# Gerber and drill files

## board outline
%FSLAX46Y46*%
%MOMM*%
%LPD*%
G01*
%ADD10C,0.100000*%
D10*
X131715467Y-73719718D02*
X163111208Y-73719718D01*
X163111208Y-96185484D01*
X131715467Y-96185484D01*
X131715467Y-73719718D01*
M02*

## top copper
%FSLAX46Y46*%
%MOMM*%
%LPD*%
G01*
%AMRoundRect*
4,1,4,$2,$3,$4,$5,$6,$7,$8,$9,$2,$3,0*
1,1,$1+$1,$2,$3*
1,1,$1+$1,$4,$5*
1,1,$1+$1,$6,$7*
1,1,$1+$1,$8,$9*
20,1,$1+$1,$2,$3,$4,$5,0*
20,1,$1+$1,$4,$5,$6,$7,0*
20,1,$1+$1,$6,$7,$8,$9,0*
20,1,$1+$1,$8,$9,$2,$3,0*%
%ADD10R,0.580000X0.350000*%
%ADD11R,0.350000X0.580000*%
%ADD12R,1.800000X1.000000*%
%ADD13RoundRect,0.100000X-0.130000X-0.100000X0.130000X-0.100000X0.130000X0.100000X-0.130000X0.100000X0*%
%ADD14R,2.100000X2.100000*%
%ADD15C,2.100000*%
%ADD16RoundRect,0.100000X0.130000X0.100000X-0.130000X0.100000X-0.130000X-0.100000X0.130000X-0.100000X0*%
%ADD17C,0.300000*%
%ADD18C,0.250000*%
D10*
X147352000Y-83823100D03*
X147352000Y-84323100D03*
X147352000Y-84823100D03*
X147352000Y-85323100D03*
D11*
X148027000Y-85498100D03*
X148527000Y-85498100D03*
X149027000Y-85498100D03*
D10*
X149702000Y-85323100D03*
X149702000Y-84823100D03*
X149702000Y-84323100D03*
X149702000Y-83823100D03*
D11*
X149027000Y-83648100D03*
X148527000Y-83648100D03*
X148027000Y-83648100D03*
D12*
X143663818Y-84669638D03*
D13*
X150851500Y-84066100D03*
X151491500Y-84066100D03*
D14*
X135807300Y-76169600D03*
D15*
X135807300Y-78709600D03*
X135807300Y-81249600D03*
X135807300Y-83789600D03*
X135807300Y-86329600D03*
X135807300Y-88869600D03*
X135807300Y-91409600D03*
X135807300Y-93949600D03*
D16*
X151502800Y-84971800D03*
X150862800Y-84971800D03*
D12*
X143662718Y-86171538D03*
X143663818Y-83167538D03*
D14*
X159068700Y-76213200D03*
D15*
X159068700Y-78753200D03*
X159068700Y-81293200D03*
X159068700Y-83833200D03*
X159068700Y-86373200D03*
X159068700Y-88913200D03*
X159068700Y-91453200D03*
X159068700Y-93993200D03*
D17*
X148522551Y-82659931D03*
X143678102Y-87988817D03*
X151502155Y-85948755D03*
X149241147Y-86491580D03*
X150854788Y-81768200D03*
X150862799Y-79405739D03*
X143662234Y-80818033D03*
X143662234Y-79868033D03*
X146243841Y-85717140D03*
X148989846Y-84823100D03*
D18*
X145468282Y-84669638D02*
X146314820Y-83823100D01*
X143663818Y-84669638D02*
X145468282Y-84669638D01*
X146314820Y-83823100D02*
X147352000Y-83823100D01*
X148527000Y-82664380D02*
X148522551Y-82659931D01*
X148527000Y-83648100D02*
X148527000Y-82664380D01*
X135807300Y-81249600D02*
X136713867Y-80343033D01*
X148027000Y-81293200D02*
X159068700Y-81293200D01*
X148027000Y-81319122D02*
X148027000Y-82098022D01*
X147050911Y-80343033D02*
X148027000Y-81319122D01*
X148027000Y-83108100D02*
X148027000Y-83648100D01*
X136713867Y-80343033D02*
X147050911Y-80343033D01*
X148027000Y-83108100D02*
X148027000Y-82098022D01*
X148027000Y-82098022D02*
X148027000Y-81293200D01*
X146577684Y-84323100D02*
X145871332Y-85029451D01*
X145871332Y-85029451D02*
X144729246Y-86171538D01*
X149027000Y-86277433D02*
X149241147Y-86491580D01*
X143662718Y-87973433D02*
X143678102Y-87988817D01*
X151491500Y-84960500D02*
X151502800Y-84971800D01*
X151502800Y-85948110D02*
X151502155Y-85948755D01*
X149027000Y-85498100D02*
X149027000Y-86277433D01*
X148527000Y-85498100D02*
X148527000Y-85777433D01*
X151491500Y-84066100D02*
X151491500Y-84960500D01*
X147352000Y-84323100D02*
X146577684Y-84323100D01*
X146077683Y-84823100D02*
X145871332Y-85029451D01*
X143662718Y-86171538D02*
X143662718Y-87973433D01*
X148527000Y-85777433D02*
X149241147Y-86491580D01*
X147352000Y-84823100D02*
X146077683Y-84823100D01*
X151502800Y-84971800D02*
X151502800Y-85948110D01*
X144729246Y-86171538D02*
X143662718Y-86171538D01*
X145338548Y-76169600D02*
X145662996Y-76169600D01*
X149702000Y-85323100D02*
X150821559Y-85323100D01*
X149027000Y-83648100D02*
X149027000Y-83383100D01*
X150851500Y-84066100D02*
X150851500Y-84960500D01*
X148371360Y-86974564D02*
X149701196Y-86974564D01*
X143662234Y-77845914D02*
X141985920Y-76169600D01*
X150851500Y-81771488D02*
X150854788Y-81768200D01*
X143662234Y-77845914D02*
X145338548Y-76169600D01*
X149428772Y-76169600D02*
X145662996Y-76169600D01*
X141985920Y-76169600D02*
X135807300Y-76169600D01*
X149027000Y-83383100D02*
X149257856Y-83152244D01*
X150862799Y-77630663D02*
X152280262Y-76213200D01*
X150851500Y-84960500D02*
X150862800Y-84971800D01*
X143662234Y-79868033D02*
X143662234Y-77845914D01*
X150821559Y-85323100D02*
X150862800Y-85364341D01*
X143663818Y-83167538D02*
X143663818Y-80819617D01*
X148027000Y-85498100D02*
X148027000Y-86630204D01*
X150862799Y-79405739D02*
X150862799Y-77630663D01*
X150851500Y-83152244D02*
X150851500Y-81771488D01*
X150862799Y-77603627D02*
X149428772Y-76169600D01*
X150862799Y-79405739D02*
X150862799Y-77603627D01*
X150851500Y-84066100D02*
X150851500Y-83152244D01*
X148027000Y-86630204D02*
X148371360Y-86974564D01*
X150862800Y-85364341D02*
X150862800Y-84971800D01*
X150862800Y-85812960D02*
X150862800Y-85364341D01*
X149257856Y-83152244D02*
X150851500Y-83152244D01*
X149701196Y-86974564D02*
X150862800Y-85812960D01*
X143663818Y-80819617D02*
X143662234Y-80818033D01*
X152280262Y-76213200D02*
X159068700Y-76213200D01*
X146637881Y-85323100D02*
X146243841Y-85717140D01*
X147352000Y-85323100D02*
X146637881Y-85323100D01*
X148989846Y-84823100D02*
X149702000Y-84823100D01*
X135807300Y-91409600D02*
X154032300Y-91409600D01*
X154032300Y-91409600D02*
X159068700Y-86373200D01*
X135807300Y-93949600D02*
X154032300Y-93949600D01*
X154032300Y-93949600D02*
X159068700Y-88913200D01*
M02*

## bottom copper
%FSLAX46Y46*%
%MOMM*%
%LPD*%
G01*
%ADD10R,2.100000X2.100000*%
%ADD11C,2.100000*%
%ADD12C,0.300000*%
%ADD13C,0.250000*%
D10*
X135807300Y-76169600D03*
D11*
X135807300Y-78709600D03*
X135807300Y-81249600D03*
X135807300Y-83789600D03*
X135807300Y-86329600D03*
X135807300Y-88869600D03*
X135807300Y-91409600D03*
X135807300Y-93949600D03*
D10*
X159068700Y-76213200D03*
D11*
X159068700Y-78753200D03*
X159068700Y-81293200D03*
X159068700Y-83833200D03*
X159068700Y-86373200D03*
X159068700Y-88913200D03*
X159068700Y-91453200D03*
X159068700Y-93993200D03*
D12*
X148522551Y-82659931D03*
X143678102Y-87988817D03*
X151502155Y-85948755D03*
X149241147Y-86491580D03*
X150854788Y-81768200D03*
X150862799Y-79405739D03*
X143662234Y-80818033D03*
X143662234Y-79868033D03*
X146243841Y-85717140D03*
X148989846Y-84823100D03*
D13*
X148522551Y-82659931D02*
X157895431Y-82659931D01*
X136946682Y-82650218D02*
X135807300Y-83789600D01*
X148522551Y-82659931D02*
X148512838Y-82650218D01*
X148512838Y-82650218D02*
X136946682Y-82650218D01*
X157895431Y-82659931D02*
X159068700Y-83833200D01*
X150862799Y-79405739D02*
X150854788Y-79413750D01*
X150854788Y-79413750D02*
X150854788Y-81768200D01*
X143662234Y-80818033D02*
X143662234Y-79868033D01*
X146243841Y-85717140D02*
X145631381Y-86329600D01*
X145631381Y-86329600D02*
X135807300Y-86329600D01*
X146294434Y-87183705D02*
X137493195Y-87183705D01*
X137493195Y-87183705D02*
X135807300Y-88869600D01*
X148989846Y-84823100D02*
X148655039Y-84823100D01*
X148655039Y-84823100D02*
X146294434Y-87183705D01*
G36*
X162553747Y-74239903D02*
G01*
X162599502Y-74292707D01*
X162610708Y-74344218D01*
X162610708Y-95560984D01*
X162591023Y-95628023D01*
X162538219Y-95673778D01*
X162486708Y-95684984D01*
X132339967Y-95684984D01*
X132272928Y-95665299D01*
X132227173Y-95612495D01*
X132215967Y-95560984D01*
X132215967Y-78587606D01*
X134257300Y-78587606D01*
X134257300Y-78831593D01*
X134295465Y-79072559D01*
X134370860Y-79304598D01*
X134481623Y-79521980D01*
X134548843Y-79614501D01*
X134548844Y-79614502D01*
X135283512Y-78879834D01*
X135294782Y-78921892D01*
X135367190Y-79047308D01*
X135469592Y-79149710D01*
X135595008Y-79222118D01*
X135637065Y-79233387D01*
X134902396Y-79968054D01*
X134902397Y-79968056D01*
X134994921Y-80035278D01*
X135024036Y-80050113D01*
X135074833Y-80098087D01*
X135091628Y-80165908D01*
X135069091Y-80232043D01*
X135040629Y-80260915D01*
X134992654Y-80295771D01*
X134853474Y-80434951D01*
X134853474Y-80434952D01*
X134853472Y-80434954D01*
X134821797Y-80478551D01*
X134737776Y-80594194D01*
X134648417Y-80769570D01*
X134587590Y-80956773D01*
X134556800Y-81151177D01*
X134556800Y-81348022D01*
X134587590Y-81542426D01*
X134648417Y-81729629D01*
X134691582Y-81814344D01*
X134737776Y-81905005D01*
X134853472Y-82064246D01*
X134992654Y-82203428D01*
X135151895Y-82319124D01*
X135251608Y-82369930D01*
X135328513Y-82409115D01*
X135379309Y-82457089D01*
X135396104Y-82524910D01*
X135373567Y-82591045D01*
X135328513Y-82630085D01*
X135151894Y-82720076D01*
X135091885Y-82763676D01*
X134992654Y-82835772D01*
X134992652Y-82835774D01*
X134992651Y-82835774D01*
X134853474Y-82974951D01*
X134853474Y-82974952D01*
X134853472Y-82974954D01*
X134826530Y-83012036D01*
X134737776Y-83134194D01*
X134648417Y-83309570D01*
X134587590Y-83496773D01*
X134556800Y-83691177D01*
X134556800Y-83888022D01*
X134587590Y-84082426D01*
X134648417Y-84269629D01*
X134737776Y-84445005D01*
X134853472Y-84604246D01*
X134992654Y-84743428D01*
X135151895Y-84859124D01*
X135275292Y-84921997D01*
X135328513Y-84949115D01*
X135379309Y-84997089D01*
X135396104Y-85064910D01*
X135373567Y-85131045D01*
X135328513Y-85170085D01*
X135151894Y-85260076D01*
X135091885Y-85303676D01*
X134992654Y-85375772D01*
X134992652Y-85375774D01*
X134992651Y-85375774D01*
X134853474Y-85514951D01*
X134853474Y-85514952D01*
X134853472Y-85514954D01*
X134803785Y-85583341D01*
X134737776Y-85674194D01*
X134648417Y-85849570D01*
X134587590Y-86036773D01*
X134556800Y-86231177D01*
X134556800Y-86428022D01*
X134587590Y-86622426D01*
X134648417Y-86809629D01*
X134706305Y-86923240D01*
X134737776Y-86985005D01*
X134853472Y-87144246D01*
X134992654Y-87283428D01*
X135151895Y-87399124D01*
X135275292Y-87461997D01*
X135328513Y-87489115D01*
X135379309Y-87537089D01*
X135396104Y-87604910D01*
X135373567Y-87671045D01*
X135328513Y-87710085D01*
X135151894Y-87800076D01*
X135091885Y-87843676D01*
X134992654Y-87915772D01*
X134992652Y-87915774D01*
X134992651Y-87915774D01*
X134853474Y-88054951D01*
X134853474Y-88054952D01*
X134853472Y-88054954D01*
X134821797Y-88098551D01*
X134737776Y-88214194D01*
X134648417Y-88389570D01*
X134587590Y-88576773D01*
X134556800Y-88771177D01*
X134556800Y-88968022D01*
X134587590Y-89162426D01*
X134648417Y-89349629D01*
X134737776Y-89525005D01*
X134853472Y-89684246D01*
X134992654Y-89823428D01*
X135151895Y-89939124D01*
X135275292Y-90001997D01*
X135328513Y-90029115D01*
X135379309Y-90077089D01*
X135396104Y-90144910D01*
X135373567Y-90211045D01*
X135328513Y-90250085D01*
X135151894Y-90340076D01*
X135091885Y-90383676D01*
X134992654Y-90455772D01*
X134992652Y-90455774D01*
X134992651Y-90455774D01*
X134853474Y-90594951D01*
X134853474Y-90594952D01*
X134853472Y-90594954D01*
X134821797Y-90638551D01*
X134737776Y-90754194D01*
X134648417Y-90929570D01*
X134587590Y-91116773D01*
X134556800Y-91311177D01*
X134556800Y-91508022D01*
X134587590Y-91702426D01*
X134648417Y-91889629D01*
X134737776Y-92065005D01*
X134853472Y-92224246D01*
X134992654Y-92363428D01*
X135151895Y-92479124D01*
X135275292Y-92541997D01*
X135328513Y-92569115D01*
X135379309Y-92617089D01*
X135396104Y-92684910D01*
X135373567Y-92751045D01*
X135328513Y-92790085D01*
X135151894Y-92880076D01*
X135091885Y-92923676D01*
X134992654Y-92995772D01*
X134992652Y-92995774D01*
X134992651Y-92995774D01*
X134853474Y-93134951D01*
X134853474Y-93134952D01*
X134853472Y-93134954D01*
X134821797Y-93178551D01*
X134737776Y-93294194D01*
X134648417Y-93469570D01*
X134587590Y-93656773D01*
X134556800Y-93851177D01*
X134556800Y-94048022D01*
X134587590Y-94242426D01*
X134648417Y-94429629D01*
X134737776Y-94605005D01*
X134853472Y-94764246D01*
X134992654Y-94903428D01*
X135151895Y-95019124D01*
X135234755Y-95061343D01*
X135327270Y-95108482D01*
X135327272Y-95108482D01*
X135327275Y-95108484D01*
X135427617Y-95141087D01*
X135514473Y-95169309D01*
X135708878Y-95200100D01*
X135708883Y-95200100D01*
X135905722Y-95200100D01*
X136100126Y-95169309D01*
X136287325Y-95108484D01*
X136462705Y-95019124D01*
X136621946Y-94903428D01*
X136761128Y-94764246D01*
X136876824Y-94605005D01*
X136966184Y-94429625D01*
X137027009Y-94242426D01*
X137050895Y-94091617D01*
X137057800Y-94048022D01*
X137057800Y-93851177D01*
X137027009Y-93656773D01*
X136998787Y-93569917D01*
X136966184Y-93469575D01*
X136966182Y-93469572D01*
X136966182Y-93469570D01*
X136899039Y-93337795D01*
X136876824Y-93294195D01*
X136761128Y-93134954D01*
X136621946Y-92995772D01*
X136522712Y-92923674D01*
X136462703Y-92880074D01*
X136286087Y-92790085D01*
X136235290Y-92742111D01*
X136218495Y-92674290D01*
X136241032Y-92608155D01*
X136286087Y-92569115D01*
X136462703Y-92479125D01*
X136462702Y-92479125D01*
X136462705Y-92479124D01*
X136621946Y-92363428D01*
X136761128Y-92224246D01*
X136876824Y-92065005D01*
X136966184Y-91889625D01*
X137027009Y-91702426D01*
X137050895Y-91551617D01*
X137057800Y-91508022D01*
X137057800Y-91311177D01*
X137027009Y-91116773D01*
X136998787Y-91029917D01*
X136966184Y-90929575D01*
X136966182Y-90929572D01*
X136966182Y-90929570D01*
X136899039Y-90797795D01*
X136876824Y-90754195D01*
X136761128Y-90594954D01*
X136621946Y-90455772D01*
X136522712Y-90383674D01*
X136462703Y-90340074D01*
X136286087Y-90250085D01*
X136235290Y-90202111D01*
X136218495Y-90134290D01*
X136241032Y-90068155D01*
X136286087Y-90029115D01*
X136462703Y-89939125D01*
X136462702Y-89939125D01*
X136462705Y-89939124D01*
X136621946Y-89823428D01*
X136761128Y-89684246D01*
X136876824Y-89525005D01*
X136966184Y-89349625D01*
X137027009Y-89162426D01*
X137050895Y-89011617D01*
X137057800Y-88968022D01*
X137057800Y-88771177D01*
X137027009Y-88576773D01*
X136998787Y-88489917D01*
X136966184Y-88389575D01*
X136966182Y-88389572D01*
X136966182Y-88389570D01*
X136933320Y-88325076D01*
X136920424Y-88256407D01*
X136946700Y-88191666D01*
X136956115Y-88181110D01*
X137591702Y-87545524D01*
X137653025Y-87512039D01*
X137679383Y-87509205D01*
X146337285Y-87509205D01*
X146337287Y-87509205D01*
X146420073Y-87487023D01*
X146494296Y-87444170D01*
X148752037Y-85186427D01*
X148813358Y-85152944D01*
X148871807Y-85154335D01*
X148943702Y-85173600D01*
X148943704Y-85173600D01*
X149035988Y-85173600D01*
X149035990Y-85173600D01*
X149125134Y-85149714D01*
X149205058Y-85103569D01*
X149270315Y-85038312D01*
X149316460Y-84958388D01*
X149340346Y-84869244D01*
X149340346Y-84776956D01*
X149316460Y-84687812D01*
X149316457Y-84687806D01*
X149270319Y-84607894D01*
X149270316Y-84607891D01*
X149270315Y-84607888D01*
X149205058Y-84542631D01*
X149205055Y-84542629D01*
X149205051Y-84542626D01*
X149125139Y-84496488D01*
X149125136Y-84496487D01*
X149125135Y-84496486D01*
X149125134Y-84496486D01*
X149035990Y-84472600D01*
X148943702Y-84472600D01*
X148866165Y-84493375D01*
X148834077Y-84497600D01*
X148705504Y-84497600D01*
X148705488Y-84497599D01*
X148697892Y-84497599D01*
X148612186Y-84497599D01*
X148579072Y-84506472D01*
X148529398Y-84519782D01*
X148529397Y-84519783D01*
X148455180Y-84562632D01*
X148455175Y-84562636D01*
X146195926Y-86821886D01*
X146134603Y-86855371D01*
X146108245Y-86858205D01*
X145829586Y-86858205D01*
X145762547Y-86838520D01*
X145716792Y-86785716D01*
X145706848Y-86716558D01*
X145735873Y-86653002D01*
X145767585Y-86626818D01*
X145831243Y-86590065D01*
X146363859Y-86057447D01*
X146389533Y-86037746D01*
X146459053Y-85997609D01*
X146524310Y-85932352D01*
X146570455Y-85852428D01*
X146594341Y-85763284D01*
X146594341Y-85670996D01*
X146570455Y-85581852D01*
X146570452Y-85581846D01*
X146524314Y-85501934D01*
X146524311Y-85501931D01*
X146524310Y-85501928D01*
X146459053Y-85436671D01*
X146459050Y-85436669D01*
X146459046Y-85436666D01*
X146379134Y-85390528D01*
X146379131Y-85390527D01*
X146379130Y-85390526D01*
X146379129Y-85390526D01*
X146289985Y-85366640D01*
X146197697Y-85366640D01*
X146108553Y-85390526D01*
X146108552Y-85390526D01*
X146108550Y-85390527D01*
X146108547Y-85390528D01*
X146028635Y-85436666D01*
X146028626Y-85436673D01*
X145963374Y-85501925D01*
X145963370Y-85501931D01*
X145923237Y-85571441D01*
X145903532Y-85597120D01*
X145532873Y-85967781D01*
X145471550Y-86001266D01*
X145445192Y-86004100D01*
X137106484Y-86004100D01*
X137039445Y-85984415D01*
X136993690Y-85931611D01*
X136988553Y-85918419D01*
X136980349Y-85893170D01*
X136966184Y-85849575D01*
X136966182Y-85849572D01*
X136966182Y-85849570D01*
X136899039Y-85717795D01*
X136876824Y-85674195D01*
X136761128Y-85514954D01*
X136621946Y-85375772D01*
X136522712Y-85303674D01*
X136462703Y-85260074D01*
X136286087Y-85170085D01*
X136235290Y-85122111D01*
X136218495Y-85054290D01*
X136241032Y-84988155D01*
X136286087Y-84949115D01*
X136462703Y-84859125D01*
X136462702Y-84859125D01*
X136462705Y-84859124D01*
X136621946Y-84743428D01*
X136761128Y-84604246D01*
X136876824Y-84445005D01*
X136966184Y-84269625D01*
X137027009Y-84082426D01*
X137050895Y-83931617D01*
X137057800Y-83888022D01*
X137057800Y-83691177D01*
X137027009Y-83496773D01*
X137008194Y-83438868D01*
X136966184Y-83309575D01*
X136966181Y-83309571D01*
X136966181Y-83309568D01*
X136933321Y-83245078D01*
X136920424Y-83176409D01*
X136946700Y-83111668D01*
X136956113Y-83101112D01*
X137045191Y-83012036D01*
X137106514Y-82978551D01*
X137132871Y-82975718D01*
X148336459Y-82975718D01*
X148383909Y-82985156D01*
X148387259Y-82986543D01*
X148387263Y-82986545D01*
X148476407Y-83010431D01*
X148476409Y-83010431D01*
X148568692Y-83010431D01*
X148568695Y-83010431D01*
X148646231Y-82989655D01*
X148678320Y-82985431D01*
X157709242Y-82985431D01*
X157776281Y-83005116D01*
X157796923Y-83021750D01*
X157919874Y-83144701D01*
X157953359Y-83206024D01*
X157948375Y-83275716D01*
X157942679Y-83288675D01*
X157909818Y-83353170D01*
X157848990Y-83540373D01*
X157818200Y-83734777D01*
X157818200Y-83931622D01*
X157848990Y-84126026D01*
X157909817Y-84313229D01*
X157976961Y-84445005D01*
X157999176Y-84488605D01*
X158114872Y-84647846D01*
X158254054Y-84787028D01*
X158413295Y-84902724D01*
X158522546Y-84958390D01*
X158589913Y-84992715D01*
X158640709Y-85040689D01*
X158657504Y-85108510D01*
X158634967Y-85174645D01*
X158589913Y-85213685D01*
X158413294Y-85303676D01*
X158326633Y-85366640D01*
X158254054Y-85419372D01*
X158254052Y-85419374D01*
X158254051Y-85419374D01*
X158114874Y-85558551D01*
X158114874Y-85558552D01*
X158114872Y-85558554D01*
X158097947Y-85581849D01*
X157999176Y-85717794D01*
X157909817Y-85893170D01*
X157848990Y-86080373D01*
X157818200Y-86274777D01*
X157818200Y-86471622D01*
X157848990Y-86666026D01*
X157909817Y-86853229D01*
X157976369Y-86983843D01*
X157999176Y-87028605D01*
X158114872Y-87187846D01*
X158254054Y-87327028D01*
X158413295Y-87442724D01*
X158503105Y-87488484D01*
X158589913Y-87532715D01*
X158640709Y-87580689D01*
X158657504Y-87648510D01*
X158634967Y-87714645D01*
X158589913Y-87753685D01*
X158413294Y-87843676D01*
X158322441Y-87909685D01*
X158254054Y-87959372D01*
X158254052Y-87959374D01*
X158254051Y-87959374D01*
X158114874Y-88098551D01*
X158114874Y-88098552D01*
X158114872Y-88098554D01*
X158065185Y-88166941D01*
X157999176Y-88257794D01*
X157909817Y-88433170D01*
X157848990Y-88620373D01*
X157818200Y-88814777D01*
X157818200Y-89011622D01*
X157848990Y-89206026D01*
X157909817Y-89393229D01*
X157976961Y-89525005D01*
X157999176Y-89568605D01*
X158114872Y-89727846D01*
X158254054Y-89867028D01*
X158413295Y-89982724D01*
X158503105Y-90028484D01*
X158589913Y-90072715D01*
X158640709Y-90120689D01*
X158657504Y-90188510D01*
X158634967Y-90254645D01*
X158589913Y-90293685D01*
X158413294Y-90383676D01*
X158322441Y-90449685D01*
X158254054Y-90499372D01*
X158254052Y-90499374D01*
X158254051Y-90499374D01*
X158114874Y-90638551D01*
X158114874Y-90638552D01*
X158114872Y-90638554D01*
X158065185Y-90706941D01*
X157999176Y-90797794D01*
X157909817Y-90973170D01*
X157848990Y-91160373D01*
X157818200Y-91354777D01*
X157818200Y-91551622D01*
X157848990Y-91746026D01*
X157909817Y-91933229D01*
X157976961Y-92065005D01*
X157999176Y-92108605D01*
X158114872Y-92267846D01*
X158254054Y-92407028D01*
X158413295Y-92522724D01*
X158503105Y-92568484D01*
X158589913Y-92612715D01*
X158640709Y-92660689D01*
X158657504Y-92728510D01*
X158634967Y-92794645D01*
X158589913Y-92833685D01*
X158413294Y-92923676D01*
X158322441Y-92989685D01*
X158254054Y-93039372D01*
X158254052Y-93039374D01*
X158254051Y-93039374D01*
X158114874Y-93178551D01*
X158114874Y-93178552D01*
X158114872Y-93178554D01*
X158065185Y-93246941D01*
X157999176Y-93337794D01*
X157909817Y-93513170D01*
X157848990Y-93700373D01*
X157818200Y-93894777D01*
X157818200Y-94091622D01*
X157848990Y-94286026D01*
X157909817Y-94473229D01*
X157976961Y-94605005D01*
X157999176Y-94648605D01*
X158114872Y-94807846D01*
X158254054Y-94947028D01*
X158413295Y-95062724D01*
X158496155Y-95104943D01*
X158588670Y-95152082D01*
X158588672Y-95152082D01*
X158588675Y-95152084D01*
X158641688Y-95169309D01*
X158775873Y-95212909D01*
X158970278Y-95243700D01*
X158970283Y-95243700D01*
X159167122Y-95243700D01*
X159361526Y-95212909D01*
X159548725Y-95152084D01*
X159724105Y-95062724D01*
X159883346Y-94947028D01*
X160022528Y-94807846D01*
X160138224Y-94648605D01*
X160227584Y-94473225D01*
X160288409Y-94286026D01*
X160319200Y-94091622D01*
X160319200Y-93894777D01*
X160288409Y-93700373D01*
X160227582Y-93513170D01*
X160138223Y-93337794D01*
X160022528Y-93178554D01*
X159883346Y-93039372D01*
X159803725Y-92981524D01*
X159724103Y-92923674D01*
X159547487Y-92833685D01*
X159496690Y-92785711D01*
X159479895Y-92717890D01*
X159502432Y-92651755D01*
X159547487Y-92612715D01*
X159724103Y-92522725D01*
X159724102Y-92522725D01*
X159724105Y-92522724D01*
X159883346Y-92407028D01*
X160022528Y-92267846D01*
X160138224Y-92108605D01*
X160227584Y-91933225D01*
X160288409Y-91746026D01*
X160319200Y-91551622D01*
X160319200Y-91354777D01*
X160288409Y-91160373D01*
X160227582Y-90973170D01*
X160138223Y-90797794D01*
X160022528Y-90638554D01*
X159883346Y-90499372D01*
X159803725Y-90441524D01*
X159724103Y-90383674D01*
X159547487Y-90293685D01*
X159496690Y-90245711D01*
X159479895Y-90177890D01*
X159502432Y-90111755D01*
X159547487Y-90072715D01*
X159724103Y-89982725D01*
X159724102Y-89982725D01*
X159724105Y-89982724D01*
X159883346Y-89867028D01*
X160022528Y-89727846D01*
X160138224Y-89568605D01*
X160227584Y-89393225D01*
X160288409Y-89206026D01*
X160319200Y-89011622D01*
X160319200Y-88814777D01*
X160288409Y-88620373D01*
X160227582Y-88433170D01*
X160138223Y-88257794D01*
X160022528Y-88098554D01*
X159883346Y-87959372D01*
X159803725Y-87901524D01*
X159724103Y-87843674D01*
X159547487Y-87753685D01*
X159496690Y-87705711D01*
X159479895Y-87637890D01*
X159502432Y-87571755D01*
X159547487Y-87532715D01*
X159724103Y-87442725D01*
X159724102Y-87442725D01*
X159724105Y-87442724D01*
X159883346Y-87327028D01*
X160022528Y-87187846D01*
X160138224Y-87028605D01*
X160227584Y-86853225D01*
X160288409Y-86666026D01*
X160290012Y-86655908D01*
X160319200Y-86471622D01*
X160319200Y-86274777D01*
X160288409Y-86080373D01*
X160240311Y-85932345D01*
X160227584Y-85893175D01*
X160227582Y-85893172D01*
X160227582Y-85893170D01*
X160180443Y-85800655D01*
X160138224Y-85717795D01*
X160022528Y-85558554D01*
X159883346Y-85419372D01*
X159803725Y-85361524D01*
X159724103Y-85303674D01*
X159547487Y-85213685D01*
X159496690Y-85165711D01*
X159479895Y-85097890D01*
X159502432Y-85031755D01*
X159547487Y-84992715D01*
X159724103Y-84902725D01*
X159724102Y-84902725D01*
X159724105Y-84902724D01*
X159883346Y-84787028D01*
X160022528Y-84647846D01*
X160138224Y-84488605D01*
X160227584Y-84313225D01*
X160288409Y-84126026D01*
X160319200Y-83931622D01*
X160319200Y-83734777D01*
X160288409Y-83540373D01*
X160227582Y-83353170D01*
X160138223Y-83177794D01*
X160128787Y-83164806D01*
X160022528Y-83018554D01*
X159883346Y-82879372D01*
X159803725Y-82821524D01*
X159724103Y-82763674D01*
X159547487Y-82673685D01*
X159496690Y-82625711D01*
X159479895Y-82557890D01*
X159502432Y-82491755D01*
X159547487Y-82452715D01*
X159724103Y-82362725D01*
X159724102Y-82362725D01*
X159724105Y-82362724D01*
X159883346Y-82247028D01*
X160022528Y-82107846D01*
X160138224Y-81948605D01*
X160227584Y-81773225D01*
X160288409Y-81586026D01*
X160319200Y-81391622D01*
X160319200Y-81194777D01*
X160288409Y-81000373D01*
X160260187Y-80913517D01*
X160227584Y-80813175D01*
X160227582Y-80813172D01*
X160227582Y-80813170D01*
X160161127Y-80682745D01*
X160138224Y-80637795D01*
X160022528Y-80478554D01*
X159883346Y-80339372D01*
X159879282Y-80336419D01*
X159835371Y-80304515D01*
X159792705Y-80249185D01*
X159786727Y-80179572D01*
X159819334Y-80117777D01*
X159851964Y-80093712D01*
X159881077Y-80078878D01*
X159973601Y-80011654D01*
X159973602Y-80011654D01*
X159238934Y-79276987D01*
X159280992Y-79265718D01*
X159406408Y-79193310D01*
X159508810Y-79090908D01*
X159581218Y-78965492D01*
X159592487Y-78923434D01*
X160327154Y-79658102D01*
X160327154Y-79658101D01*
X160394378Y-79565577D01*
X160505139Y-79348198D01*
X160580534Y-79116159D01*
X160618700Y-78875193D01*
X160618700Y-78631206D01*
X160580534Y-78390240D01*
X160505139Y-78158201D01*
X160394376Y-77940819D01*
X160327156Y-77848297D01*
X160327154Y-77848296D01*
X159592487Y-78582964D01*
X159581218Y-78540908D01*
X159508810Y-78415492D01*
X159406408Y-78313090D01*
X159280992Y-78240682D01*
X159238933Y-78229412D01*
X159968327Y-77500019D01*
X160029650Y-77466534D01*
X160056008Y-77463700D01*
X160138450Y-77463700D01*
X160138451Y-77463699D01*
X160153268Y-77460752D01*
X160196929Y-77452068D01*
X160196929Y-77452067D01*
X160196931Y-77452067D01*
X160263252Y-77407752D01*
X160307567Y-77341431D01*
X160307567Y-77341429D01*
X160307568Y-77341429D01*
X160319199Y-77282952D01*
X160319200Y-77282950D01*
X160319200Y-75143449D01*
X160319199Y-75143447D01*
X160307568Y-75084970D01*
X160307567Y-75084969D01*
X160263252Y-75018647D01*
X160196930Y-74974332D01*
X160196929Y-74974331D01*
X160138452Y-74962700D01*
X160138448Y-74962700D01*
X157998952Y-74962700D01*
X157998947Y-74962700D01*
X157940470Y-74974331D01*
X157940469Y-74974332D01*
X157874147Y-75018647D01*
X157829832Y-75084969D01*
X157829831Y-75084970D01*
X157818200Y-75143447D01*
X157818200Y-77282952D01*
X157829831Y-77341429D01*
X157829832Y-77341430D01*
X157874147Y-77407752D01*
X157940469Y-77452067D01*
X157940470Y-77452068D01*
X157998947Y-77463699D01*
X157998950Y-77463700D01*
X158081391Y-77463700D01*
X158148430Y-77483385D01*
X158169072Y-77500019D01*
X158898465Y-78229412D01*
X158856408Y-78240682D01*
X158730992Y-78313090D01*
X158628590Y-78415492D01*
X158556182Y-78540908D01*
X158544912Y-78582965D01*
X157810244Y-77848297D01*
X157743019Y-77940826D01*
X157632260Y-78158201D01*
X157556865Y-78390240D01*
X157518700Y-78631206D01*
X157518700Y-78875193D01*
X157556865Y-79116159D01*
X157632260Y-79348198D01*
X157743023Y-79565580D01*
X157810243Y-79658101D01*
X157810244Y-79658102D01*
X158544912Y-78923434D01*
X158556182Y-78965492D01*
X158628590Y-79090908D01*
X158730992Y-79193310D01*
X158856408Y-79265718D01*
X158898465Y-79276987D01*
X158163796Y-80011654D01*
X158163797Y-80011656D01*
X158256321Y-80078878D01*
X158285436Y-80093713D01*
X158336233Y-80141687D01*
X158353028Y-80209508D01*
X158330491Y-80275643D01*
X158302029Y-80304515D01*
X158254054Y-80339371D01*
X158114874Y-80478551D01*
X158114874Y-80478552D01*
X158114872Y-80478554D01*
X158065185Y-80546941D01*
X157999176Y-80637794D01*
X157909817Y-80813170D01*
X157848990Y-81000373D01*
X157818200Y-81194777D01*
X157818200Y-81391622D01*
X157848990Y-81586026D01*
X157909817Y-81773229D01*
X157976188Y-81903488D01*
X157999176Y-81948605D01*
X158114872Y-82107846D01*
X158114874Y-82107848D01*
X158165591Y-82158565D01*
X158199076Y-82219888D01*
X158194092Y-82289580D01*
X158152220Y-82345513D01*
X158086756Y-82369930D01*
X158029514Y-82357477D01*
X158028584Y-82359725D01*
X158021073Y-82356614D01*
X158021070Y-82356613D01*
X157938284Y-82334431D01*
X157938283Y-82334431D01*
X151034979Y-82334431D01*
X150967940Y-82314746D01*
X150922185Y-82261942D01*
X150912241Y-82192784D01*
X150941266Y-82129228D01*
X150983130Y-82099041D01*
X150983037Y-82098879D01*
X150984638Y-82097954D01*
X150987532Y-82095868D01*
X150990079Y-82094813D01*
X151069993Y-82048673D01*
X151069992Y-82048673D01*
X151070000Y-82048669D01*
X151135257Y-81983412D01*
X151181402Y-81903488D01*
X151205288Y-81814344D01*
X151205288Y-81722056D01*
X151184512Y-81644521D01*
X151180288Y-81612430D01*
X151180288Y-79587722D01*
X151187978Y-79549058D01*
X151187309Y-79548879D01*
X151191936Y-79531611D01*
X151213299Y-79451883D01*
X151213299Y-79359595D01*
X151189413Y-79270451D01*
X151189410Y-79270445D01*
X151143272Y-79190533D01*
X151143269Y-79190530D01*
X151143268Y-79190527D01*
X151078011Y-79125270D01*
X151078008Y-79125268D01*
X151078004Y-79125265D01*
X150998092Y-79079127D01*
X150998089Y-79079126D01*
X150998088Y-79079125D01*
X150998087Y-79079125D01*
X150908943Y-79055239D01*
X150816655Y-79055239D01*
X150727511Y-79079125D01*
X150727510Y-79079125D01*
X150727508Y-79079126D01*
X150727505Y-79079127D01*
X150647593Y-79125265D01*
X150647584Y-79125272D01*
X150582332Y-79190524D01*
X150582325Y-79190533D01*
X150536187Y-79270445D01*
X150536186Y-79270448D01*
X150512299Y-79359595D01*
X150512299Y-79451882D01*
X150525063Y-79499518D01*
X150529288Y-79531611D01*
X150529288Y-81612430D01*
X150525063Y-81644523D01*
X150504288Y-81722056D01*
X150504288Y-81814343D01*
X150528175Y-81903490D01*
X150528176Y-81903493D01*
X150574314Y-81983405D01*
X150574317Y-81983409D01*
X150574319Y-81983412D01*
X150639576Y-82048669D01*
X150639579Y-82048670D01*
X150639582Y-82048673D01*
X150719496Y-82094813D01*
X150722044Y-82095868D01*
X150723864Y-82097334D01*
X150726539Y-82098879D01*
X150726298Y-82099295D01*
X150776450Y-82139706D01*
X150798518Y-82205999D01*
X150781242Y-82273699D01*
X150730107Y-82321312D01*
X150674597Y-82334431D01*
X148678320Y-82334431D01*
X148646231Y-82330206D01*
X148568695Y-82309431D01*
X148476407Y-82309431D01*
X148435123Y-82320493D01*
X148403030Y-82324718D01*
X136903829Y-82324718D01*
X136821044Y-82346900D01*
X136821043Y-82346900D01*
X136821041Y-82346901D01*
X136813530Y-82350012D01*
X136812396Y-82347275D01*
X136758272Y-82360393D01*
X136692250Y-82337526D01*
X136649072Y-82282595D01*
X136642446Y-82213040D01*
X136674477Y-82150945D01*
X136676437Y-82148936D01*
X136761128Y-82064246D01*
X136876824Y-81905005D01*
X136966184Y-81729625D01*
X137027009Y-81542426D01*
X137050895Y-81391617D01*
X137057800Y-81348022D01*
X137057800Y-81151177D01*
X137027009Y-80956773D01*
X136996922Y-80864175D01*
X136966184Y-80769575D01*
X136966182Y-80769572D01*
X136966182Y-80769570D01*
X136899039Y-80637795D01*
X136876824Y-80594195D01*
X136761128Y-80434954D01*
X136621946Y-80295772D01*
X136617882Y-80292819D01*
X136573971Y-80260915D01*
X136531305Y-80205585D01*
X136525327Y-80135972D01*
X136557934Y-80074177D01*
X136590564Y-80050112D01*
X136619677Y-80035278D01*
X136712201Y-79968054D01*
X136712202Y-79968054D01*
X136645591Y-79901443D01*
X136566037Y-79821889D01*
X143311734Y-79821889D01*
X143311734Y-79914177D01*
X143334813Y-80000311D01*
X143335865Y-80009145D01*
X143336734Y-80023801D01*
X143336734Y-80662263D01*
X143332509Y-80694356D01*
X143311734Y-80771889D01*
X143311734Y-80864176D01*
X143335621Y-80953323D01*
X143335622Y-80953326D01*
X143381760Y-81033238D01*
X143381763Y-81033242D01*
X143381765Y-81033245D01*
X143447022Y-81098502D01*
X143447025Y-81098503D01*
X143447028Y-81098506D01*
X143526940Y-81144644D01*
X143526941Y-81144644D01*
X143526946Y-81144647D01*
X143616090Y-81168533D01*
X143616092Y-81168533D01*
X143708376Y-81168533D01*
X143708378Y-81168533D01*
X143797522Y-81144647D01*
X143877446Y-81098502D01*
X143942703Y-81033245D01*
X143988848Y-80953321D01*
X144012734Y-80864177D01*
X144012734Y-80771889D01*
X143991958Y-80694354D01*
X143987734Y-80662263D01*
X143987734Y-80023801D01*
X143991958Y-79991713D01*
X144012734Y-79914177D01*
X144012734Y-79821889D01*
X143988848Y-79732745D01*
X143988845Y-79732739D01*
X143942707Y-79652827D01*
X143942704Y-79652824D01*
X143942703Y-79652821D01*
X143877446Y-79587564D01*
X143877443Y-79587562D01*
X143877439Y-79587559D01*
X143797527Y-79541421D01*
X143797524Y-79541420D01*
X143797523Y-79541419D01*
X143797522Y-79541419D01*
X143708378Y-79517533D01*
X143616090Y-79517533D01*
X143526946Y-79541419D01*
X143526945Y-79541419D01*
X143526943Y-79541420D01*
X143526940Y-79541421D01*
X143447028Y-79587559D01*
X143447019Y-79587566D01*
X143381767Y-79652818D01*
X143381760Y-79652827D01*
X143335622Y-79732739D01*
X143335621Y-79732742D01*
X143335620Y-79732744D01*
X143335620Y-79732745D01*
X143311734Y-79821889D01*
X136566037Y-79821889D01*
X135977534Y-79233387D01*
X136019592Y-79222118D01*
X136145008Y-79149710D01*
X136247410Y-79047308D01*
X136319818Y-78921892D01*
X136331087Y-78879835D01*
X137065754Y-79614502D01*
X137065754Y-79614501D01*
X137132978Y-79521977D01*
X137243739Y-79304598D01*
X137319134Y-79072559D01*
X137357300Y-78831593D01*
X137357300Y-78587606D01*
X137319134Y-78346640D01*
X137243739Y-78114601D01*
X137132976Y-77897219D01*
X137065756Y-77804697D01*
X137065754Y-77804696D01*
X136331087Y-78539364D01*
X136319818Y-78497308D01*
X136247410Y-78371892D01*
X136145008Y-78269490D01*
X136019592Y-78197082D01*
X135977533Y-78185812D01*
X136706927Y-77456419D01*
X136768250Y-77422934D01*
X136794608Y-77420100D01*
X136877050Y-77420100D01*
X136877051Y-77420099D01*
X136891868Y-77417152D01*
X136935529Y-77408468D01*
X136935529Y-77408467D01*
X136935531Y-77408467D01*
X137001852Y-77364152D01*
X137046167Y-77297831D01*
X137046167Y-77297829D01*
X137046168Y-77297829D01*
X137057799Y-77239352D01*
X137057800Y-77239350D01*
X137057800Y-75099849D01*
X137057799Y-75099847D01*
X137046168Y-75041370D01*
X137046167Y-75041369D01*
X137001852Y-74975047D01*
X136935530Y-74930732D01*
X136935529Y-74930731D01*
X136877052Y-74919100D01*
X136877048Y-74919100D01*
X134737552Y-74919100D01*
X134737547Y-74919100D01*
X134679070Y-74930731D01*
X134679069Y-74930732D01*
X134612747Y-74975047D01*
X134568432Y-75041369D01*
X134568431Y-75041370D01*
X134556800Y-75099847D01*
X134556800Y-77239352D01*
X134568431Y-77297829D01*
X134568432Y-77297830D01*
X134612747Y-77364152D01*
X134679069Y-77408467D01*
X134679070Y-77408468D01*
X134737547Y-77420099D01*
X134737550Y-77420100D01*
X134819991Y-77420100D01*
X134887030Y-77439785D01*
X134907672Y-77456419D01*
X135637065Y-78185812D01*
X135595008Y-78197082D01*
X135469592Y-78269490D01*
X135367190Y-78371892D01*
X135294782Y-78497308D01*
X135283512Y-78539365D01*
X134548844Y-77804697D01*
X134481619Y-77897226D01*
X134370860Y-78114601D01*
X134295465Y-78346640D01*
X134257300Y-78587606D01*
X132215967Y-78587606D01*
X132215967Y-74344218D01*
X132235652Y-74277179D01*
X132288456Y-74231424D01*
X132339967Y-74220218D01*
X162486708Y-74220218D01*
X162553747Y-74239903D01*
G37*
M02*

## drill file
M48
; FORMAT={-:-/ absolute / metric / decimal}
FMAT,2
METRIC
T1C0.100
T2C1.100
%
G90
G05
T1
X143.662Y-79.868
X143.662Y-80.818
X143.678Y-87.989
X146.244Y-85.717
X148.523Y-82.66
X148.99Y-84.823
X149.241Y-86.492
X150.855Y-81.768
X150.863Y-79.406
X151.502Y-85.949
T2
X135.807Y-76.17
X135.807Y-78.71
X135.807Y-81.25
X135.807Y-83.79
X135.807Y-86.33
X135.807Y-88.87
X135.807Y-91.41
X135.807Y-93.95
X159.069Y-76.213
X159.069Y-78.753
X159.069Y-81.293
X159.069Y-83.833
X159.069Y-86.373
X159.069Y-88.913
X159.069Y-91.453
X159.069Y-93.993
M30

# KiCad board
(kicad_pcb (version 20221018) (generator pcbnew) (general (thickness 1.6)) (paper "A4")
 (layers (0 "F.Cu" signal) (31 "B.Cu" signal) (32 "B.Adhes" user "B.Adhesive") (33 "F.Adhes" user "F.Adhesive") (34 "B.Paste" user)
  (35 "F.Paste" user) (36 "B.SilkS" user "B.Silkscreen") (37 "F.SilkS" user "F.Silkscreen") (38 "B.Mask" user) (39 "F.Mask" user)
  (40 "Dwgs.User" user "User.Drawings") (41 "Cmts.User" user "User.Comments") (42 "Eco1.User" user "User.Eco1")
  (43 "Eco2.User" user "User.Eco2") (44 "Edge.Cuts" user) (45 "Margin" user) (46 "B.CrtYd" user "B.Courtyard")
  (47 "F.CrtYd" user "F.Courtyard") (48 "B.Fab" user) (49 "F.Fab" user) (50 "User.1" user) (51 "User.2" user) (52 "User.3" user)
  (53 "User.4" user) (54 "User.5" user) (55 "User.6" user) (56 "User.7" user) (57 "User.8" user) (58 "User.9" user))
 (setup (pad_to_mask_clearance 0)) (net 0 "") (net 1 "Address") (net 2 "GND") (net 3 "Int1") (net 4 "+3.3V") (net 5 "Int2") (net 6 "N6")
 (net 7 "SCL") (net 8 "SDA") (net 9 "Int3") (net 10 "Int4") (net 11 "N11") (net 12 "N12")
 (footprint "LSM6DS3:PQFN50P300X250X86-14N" (layer "F.Cu") (at 148.527 84.5731)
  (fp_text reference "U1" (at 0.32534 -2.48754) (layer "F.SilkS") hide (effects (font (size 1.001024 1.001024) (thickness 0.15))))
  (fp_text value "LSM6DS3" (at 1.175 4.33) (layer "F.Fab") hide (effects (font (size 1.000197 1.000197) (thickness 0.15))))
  (pad "1" smd rect (at -1.175 -0.75 180) (size 0.58 0.35) (layers "F.Cu" "F.Paste" "F.Mask") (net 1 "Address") (solder_mask_margin 0.102))
  (pad "2" smd rect (at -1.175 -0.25 180) (size 0.58 0.35) (layers "F.Cu" "F.Paste" "F.Mask") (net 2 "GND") (solder_mask_margin 0.102))
  (pad "3" smd rect (at -1.175 0.25 180) (size 0.58 0.35) (layers "F.Cu" "F.Paste" "F.Mask") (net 2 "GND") (solder_mask_margin 0.102))
  (pad "4" smd rect (at -1.175 0.75 180) (size 0.58 0.35) (layers "F.Cu" "F.Paste" "F.Mask") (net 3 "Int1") (solder_mask_margin 0.102))
  (pad "5" smd rect (at -0.5 0.925 90) (size 0.58 0.35) (layers "F.Cu" "F.Paste" "F.Mask") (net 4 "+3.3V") (solder_mask_margin 0.102))
  (pad "6" smd rect (at 0 0.925 90) (size 0.58 0.35) (layers "F.Cu" "F.Paste" "F.Mask") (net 2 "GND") (solder_mask_margin 0.102))
  (pad "7" smd rect (at 0.5 0.925 90) (size 0.58 0.35) (layers "F.Cu" "F.Paste" "F.Mask") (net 2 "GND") (solder_mask_margin 0.102))
  (pad "8" smd rect (at 1.175 0.75 180) (size 0.58 0.35) (layers "F.Cu" "F.Paste" "F.Mask") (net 4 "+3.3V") (solder_mask_margin 0.102))
  (pad "9" smd rect (at 1.175 0.25 180) (size 0.58 0.35) (layers "F.Cu" "F.Paste" "F.Mask") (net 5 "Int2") (solder_mask_margin 0.102))
  (pad "10" smd rect (at 1.175 -0.25 180) (size 0.58 0.35) (layers "F.Cu" "F.Paste" "F.Mask") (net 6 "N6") (solder_mask_margin 0.102))
  (pad "11" smd rect (at 1.175 -0.75 180) (size 0.58 0.35) (layers "F.Cu" "F.Paste" "F.Mask") (solder_mask_margin 0.102))
  (pad "12" smd rect (at 0.5 -0.925 90) (size 0.58 0.35) (layers "F.Cu" "F.Paste" "F.Mask") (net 4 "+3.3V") (solder_mask_margin 0.102))
  (pad "13" smd rect (at 0 -0.925 90) (size 0.58 0.35) (layers "F.Cu" "F.Paste" "F.Mask") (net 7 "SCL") (solder_mask_margin 0.102))
  (pad "14" smd rect (at -0.5 -0.925 90) (size 0.58 0.35) (layers "F.Cu" "F.Paste" "F.Mask") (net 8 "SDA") (solder_mask_margin 0.102)))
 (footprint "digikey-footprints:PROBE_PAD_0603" (layer "F.Cu") (at 143.663818 84.669638)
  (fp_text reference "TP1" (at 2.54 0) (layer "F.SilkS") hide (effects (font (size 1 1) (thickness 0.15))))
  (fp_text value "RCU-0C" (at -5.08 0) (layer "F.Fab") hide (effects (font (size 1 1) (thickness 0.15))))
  (pad "1" smd rect (at 0 0) (size 1.8 1) (layers "F.Cu" "F.Paste" "F.Mask") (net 1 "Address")))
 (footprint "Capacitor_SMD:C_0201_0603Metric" (layer "F.Cu") (at 151.1715 84.0661)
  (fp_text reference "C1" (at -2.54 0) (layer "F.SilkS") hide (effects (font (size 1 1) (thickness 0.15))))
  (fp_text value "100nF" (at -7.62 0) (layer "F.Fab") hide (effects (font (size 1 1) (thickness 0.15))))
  (pad "" smd roundrect (at -0.345 0) (size 0.318 0.36) (layers "F.Paste") (roundrect_rratio 0.25))
  (pad "" smd roundrect (at 0.345 0) (size 0.318 0.36) (layers "F.Paste") (roundrect_rratio 0.25))
  (pad "1" smd roundrect (at -0.32 0) (size 0.46 0.4) (layers "F.Cu" "F.Mask") (roundrect_rratio 0.25) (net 4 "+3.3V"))
  (pad "2" smd roundrect (at 0.32 0) (size 0.46 0.4) (layers "F.Cu" "F.Mask") (roundrect_rratio 0.25) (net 2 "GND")))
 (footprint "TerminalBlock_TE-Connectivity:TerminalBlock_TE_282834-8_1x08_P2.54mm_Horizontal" (layer "F.Cu") (at 135.8073 76.1696 -90)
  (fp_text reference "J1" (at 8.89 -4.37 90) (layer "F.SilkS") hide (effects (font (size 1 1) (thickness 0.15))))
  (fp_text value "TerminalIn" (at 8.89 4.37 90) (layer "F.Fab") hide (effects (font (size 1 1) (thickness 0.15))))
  (pad "1" thru_hole rect (at 0 0 270) (size 2.1 2.1) (drill 1.1) (layers "*.Cu" "*.Mask") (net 4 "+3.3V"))
  (pad "2" thru_hole circle (at 2.54 0 270) (size 2.1 2.1) (drill 1.1) (layers "*.Cu" "*.Mask") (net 2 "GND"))
  (pad "3" thru_hole circle (at 5.08 0 270) (size 2.1 2.1) (drill 1.1) (layers "*.Cu" "*.Mask") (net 8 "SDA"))
  (pad "4" thru_hole circle (at 7.62 0 270) (size 2.1 2.1) (drill 1.1) (layers "*.Cu" "*.Mask") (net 7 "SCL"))
  (pad "5" thru_hole circle (at 10.16 0 270) (size 2.1 2.1) (drill 1.1) (layers "*.Cu" "*.Mask") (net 3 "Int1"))
  (pad "6" thru_hole circle (at 12.7 0 270) (size 2.1 2.1) (drill 1.1) (layers "*.Cu" "*.Mask") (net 5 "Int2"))
  (pad "7" thru_hole circle (at 15.24 0 270) (size 2.1 2.1) (drill 1.1) (layers "*.Cu" "*.Mask") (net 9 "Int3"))
  (pad "8" thru_hole circle (at 17.78 0 270) (size 2.1 2.1) (drill 1.1) (layers "*.Cu" "*.Mask") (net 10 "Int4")))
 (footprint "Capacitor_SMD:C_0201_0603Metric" (layer "F.Cu") (at 151.1828 84.9718 180)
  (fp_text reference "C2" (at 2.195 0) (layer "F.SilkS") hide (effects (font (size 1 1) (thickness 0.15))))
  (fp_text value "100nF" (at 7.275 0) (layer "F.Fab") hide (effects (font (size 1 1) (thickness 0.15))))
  (pad "" smd roundrect (at -0.345 0 180) (size 0.318 0.36) (layers "F.Paste") (roundrect_rratio 0.25))
  (pad "" smd roundrect (at 0.345 0 180) (size 0.318 0.36) (layers "F.Paste") (roundrect_rratio 0.25))
  (pad "1" smd roundrect (at -0.32 0 180) (size 0.46 0.4) (layers "F.Cu" "F.Mask") (roundrect_rratio 0.25) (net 2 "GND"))
  (pad "2" smd roundrect (at 0.32 0 180) (size 0.46 0.4) (layers "F.Cu" "F.Mask") (roundrect_rratio 0.25) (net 4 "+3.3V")))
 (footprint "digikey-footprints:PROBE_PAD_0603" (layer "F.Cu") (at 143.662718 86.171538)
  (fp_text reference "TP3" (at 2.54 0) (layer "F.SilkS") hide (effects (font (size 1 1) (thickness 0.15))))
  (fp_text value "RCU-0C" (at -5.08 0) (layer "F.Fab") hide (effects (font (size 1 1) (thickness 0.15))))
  (pad "1" smd rect (at 0 0) (size 1.8 1) (layers "F.Cu" "F.Paste" "F.Mask") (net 2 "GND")))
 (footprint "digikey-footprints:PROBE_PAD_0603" (layer "F.Cu") (at 143.663818 83.167538)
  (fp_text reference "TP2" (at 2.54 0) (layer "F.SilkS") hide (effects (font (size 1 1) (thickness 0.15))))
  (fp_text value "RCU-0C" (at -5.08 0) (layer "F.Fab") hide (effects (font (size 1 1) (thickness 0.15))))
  (pad "1" smd rect (at 0 0) (size 1.8 1) (layers "F.Cu" "F.Paste" "F.Mask") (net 4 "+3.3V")))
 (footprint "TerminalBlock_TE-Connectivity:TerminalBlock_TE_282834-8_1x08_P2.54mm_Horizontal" (layer "F.Cu") (at 159.0687 76.2132 -90)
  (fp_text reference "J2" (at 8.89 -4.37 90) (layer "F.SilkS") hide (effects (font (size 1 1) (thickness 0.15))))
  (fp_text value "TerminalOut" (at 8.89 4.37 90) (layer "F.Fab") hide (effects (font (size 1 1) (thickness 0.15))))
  (pad "1" thru_hole rect (at 0 0 270) (size 2.1 2.1) (drill 1.1) (layers "*.Cu" "*.Mask") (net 4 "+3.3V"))
  (pad "2" thru_hole circle (at 2.54 0 270) (size 2.1 2.1) (drill 1.1) (layers "*.Cu" "*.Mask") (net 2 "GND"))
  (pad "3" thru_hole circle (at 5.08 0 270) (size 2.1 2.1) (drill 1.1) (layers "*.Cu" "*.Mask") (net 8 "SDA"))
  (pad "4" thru_hole circle (at 7.62 0 270) (size 2.1 2.1) (drill 1.1) (layers "*.Cu" "*.Mask") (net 7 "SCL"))
  (pad "5" thru_hole circle (at 10.16 0 270) (size 2.1 2.1) (drill 1.1) (layers "*.Cu" "*.Mask") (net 9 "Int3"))
  (pad "6" thru_hole circle (at 12.7 0 270) (size 2.1 2.1) (drill 1.1) (layers "*.Cu" "*.Mask") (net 10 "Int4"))
  (pad "7" thru_hole circle (at 15.24 0 270) (size 2.1 2.1) (drill 1.1) (layers "*.Cu" "*.Mask") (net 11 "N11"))
  (pad "8" thru_hole circle (at 17.78 0 270) (size 2.1 2.1) (drill 1.1) (layers "*.Cu" "*.Mask") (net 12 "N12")))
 (gr_rect (start 131.715467 73.719718) (end 163.111208 96.185484) (stroke (width 0.1) (type default)) (fill none) (layer "Edge.Cuts"))
 (segment (start 145.468282 84.669638) (end 146.31482 83.8231) (width 0.25) (layer "F.Cu") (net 1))
 (segment (start 143.663818 84.669638) (end 145.468282 84.669638) (width 0.25) (layer "F.Cu") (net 1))
 (segment (start 146.31482 83.8231) (end 147.352 83.8231) (width 0.25) (layer "F.Cu") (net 1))
 (segment (start 148.527 82.66438) (end 148.522551 82.659931) (width 0.25) (layer "F.Cu") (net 7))
 (segment (start 148.527 83.6481) (end 148.527 82.66438) (width 0.25) (layer "F.Cu") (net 7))
 (via micro (at 148.522551 82.659931) (size 0.3) (drill 0.1) (layers "F.Cu" "B.Cu") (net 7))
 (segment (start 148.522551 82.659931) (end 157.895431 82.659931) (width 0.25) (layer "B.Cu") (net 7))
 (segment (start 136.946682 82.650218) (end 135.8073 83.7896) (width 0.25) (layer "B.Cu") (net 7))
 (segment (start 148.522551 82.659931) (end 148.512838 82.650218) (width 0.25) (layer "B.Cu") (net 7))
 (segment (start 148.512838 82.650218) (end 136.946682 82.650218) (width 0.25) (layer "B.Cu") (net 7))
 (segment (start 157.895431 82.659931) (end 159.0687 83.8332) (width 0.25) (layer "B.Cu") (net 7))
 (segment (start 135.8073 81.2496) (end 136.713867 80.343033) (width 0.25) (layer "F.Cu") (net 8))
 (segment (start 148.027 81.2932) (end 159.0687 81.2932) (width 0.25) (layer "F.Cu") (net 8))
 (segment (start 148.027 81.319122) (end 148.027 82.098022) (width 0.25) (layer "F.Cu") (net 8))
 (segment (start 147.050911 80.343033) (end 148.027 81.319122) (width 0.25) (layer "F.Cu") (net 8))
 (segment (start 148.027 83.1081) (end 148.027 83.6481) (width 0.25) (layer "F.Cu") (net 8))
 (segment (start 136.713867 80.343033) (end 147.050911 80.343033) (width 0.25) (layer "F.Cu") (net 8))
 (segment (start 148.027 83.1081) (end 148.027 82.098022) (width 0.25) (layer "F.Cu") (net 8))
 (segment (start 148.027 82.098022) (end 148.027 81.2932) (width 0.25) (layer "F.Cu") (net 8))
 (segment (start 146.577684 84.3231) (end 145.871332 85.029451) (width 0.25) (layer "F.Cu") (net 2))
 (segment (start 145.871332 85.029451) (end 144.729246 86.171538) (width 0.25) (layer "F.Cu") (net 2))
 (segment (start 149.027 86.277433) (end 149.241147 86.49158) (width 0.25) (layer "F.Cu") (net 2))
 (segment (start 143.662718 87.973433) (end 143.678102 87.988817) (width 0.25) (layer "F.Cu") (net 2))
 (segment (start 151.4915 84.9605) (end 151.5028 84.9718) (width 0.25) (layer "F.Cu") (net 2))
 (segment (start 151.5028 85.94811) (end 151.502155 85.948755) (width 0.25) (layer "F.Cu") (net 2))
 (segment (start 149.027 85.4981) (end 149.027 86.277433) (width 0.25) (layer "F.Cu") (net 2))
 (segment (start 148.527 85.4981) (end 148.527 85.777433) (width 0.25) (layer "F.Cu") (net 2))
 (segment (start 151.4915 84.0661) (end 151.4915 84.9605) (width 0.25) (layer "F.Cu") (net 2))
 (segment (start 147.352 84.3231) (end 146.577684 84.3231) (width 0.25) (layer "F.Cu") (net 2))
 (segment (start 146.077683 84.8231) (end 145.871332 85.029451) (width 0.25) (layer "F.Cu") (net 2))
 (segment (start 143.662718 86.171538) (end 143.662718 87.973433) (width 0.25) (layer "F.Cu") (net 2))
 (segment (start 148.527 85.777433) (end 149.241147 86.49158) (width 0.25) (layer "F.Cu") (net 2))
 (segment (start 147.352 84.8231) (end 146.077683 84.8231) (width 0.25) (layer "F.Cu") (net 2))
 (segment (start 151.5028 84.9718) (end 151.5028 85.94811) (width 0.25) (layer "F.Cu") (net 2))
 (segment (start 144.729246 86.171538) (end 143.662718 86.171538) (width 0.25) (layer "F.Cu") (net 2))
 (via micro (at 143.678102 87.988817) (size 0.3) (drill 0.1) (layers "F.Cu" "B.Cu") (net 2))
 (via micro (at 151.502155 85.948755) (size 0.3) (drill 0.1) (layers "F.Cu" "B.Cu") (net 2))
 (via micro (at 149.241147 86.49158) (size 0.3) (drill 0.1) (layers "F.Cu" "B.Cu") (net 2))
 (segment (start 145.338548 76.1696) (end 145.662996 76.1696) (width 0.25) (layer "F.Cu") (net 4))
 (segment (start 149.702 85.3231) (end 150.821559 85.3231) (width 0.25) (layer "F.Cu") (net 4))
 (segment (start 149.027 83.6481) (end 149.027 83.3831) (width 0.25) (layer "F.Cu") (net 4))
 (segment (start 150.8515 84.0661) (end 150.8515 84.9605) (width 0.25) (layer "F.Cu") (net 4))
 (segment (start 148.37136 86.974564) (end 149.701196 86.974564) (width 0.25) (layer "F.Cu") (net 4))
 (segment (start 143.662234 77.845914) (end 141.98592 76.1696) (width 0.25) (layer "F.Cu") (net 4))
 (segment (start 150.8515 81.771488) (end 150.854788 81.7682) (width 0.25) (layer "F.Cu") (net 4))
 (segment (start 143.662234 77.845914) (end 145.338548 76.1696) (width 0.25) (layer "F.Cu") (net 4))
 (segment (start 149.428772 76.1696) (end 145.662996 76.1696) (width 0.25) (layer "F.Cu") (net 4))
 (segment (start 141.98592 76.1696) (end 135.8073 76.1696) (width 0.25) (layer "F.Cu") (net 4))
 (segment (start 149.027 83.3831) (end 149.257856 83.152244) (width 0.25) (layer "F.Cu") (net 4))
 (segment (start 150.862799 77.630663) (end 152.280262 76.2132) (width 0.25) (layer "F.Cu") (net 4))
 (segment (start 150.8515 84.9605) (end 150.8628 84.9718) (width 0.25) (layer "F.Cu") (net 4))
 (segment (start 143.662234 79.868033) (end 143.662234 77.845914) (width 0.25) (layer "F.Cu") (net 4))
 (segment (start 150.821559 85.3231) (end 150.8628 85.364341) (width 0.25) (layer "F.Cu") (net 4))
 (segment (start 143.663818 83.167538) (end 143.663818 80.819617) (width 0.25) (layer "F.Cu") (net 4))
 (segment (start 148.027 85.4981) (end 148.027 86.630204) (width 0.25) (layer "F.Cu") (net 4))
 (segment (start 150.862799 79.405739) (end 150.862799 77.630663) (width 0.25) (layer "F.Cu") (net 4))
 (segment (start 150.8515 83.152244) (end 150.8515 81.771488) (width 0.25) (layer "F.Cu") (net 4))
 (segment (start 150.862799 77.603627) (end 149.428772 76.1696) (width 0.25) (layer "F.Cu") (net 4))
 (segment (start 150.862799 79.405739) (end 150.862799 77.603627) (width 0.25) (layer "F.Cu") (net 4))
 (segment (start 150.8515 84.0661) (end 150.8515 83.152244) (width 0.25) (layer "F.Cu") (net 4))
 (segment (start 148.027 86.630204) (end 148.37136 86.974564) (width 0.25) (layer "F.Cu") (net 4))
 (segment (start 150.8628 85.364341) (end 150.8628 84.9718) (width 0.25) (layer "F.Cu") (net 4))
 (segment (start 150.8628 85.81296) (end 150.8628 85.364341) (width 0.25) (layer "F.Cu") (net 4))
 (segment (start 149.257856 83.152244) (end 150.8515 83.152244) (width 0.25) (layer "F.Cu") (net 4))
 (segment (start 149.701196 86.974564) (end 150.8628 85.81296) (width 0.25) (layer "F.Cu") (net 4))
 (segment (start 143.663818 80.819617) (end 143.662234 80.818033) (width 0.25) (layer "F.Cu") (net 4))
 (segment (start 152.280262 76.2132) (end 159.0687 76.2132) (width 0.25) (layer "F.Cu") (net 4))
 (via micro (at 150.854788 81.7682) (size 0.3) (drill 0.1) (layers "F.Cu" "B.Cu") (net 4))
 (via micro (at 150.862799 79.405739) (size 0.3) (drill 0.1) (layers "F.Cu" "B.Cu") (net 4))
 (via micro (at 143.662234 80.818033) (size 0.3) (drill 0.1) (layers "F.Cu" "B.Cu") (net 4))
 (via micro (at 143.662234 79.868033) (size 0.3) (drill 0.1) (layers "F.Cu" "B.Cu") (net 4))
 (segment (start 150.862799 79.405739) (end 150.854788 79.41375) (width 0.25) (layer "B.Cu") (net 4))
 (segment (start 150.854788 79.41375) (end 150.854788 81.7682) (width 0.25) (layer "B.Cu") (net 4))
 (segment (start 143.662234 80.818033) (end 143.662234 79.868033) (width 0.25) (layer "B.Cu") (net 4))
 (segment (start 146.637881 85.3231) (end 146.243841 85.71714) (width 0.25) (layer "F.Cu") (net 3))
 (segment (start 147.352 85.3231) (end 146.637881 85.3231) (width 0.25) (layer "F.Cu") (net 3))
 (via micro (at 146.243841 85.71714) (size 0.3) (drill 0.1) (layers "F.Cu" "B.Cu") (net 3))
 (segment (start 146.243841 85.71714) (end 145.631381 86.3296) (width 0.25) (layer "B.Cu") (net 3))
 (segment (start 145.631381 86.3296) (end 135.8073 86.3296) (width 0.25) (layer "B.Cu") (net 3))
 (segment (start 148.989846 84.8231) (end 149.702 84.8231) (width 0.25) (layer "F.Cu") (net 5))
 (via micro (at 148.989846 84.8231) (size 0.3) (drill 0.1) (layers "F.Cu" "B.Cu") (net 5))
 (segment (start 146.294434 87.183705) (end 137.493195 87.183705) (width 0.25) (layer "B.Cu") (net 5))
 (segment (start 137.493195 87.183705) (end 135.8073 88.8696) (width 0.25) (layer "B.Cu") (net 5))
 (segment (start 148.989846 84.8231) (end 148.655039 84.8231) (width 0.25) (layer "B.Cu") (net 5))
 (segment (start 148.655039 84.8231) (end 146.294434 87.183705) (width 0.25) (layer "B.Cu") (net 5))
 (segment (start 135.8073 91.4096) (end 154.0323 91.4096) (width 0.25) (layer "F.Cu") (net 9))
 (segment (start 154.0323 91.4096) (end 159.0687 86.3732) (width 0.25) (layer "F.Cu") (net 9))
 (segment (start 135.8073 93.9496) (end 154.0323 93.9496) (width 0.25) (layer "F.Cu") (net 10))
 (segment (start 154.0323 93.9496) (end 159.0687 88.9132) (width 0.25) (layer "F.Cu") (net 10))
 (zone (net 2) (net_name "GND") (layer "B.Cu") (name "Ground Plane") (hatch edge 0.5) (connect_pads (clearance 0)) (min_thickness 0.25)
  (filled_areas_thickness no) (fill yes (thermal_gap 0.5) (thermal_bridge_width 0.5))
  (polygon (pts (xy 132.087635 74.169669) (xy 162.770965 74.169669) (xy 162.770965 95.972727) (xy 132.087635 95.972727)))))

